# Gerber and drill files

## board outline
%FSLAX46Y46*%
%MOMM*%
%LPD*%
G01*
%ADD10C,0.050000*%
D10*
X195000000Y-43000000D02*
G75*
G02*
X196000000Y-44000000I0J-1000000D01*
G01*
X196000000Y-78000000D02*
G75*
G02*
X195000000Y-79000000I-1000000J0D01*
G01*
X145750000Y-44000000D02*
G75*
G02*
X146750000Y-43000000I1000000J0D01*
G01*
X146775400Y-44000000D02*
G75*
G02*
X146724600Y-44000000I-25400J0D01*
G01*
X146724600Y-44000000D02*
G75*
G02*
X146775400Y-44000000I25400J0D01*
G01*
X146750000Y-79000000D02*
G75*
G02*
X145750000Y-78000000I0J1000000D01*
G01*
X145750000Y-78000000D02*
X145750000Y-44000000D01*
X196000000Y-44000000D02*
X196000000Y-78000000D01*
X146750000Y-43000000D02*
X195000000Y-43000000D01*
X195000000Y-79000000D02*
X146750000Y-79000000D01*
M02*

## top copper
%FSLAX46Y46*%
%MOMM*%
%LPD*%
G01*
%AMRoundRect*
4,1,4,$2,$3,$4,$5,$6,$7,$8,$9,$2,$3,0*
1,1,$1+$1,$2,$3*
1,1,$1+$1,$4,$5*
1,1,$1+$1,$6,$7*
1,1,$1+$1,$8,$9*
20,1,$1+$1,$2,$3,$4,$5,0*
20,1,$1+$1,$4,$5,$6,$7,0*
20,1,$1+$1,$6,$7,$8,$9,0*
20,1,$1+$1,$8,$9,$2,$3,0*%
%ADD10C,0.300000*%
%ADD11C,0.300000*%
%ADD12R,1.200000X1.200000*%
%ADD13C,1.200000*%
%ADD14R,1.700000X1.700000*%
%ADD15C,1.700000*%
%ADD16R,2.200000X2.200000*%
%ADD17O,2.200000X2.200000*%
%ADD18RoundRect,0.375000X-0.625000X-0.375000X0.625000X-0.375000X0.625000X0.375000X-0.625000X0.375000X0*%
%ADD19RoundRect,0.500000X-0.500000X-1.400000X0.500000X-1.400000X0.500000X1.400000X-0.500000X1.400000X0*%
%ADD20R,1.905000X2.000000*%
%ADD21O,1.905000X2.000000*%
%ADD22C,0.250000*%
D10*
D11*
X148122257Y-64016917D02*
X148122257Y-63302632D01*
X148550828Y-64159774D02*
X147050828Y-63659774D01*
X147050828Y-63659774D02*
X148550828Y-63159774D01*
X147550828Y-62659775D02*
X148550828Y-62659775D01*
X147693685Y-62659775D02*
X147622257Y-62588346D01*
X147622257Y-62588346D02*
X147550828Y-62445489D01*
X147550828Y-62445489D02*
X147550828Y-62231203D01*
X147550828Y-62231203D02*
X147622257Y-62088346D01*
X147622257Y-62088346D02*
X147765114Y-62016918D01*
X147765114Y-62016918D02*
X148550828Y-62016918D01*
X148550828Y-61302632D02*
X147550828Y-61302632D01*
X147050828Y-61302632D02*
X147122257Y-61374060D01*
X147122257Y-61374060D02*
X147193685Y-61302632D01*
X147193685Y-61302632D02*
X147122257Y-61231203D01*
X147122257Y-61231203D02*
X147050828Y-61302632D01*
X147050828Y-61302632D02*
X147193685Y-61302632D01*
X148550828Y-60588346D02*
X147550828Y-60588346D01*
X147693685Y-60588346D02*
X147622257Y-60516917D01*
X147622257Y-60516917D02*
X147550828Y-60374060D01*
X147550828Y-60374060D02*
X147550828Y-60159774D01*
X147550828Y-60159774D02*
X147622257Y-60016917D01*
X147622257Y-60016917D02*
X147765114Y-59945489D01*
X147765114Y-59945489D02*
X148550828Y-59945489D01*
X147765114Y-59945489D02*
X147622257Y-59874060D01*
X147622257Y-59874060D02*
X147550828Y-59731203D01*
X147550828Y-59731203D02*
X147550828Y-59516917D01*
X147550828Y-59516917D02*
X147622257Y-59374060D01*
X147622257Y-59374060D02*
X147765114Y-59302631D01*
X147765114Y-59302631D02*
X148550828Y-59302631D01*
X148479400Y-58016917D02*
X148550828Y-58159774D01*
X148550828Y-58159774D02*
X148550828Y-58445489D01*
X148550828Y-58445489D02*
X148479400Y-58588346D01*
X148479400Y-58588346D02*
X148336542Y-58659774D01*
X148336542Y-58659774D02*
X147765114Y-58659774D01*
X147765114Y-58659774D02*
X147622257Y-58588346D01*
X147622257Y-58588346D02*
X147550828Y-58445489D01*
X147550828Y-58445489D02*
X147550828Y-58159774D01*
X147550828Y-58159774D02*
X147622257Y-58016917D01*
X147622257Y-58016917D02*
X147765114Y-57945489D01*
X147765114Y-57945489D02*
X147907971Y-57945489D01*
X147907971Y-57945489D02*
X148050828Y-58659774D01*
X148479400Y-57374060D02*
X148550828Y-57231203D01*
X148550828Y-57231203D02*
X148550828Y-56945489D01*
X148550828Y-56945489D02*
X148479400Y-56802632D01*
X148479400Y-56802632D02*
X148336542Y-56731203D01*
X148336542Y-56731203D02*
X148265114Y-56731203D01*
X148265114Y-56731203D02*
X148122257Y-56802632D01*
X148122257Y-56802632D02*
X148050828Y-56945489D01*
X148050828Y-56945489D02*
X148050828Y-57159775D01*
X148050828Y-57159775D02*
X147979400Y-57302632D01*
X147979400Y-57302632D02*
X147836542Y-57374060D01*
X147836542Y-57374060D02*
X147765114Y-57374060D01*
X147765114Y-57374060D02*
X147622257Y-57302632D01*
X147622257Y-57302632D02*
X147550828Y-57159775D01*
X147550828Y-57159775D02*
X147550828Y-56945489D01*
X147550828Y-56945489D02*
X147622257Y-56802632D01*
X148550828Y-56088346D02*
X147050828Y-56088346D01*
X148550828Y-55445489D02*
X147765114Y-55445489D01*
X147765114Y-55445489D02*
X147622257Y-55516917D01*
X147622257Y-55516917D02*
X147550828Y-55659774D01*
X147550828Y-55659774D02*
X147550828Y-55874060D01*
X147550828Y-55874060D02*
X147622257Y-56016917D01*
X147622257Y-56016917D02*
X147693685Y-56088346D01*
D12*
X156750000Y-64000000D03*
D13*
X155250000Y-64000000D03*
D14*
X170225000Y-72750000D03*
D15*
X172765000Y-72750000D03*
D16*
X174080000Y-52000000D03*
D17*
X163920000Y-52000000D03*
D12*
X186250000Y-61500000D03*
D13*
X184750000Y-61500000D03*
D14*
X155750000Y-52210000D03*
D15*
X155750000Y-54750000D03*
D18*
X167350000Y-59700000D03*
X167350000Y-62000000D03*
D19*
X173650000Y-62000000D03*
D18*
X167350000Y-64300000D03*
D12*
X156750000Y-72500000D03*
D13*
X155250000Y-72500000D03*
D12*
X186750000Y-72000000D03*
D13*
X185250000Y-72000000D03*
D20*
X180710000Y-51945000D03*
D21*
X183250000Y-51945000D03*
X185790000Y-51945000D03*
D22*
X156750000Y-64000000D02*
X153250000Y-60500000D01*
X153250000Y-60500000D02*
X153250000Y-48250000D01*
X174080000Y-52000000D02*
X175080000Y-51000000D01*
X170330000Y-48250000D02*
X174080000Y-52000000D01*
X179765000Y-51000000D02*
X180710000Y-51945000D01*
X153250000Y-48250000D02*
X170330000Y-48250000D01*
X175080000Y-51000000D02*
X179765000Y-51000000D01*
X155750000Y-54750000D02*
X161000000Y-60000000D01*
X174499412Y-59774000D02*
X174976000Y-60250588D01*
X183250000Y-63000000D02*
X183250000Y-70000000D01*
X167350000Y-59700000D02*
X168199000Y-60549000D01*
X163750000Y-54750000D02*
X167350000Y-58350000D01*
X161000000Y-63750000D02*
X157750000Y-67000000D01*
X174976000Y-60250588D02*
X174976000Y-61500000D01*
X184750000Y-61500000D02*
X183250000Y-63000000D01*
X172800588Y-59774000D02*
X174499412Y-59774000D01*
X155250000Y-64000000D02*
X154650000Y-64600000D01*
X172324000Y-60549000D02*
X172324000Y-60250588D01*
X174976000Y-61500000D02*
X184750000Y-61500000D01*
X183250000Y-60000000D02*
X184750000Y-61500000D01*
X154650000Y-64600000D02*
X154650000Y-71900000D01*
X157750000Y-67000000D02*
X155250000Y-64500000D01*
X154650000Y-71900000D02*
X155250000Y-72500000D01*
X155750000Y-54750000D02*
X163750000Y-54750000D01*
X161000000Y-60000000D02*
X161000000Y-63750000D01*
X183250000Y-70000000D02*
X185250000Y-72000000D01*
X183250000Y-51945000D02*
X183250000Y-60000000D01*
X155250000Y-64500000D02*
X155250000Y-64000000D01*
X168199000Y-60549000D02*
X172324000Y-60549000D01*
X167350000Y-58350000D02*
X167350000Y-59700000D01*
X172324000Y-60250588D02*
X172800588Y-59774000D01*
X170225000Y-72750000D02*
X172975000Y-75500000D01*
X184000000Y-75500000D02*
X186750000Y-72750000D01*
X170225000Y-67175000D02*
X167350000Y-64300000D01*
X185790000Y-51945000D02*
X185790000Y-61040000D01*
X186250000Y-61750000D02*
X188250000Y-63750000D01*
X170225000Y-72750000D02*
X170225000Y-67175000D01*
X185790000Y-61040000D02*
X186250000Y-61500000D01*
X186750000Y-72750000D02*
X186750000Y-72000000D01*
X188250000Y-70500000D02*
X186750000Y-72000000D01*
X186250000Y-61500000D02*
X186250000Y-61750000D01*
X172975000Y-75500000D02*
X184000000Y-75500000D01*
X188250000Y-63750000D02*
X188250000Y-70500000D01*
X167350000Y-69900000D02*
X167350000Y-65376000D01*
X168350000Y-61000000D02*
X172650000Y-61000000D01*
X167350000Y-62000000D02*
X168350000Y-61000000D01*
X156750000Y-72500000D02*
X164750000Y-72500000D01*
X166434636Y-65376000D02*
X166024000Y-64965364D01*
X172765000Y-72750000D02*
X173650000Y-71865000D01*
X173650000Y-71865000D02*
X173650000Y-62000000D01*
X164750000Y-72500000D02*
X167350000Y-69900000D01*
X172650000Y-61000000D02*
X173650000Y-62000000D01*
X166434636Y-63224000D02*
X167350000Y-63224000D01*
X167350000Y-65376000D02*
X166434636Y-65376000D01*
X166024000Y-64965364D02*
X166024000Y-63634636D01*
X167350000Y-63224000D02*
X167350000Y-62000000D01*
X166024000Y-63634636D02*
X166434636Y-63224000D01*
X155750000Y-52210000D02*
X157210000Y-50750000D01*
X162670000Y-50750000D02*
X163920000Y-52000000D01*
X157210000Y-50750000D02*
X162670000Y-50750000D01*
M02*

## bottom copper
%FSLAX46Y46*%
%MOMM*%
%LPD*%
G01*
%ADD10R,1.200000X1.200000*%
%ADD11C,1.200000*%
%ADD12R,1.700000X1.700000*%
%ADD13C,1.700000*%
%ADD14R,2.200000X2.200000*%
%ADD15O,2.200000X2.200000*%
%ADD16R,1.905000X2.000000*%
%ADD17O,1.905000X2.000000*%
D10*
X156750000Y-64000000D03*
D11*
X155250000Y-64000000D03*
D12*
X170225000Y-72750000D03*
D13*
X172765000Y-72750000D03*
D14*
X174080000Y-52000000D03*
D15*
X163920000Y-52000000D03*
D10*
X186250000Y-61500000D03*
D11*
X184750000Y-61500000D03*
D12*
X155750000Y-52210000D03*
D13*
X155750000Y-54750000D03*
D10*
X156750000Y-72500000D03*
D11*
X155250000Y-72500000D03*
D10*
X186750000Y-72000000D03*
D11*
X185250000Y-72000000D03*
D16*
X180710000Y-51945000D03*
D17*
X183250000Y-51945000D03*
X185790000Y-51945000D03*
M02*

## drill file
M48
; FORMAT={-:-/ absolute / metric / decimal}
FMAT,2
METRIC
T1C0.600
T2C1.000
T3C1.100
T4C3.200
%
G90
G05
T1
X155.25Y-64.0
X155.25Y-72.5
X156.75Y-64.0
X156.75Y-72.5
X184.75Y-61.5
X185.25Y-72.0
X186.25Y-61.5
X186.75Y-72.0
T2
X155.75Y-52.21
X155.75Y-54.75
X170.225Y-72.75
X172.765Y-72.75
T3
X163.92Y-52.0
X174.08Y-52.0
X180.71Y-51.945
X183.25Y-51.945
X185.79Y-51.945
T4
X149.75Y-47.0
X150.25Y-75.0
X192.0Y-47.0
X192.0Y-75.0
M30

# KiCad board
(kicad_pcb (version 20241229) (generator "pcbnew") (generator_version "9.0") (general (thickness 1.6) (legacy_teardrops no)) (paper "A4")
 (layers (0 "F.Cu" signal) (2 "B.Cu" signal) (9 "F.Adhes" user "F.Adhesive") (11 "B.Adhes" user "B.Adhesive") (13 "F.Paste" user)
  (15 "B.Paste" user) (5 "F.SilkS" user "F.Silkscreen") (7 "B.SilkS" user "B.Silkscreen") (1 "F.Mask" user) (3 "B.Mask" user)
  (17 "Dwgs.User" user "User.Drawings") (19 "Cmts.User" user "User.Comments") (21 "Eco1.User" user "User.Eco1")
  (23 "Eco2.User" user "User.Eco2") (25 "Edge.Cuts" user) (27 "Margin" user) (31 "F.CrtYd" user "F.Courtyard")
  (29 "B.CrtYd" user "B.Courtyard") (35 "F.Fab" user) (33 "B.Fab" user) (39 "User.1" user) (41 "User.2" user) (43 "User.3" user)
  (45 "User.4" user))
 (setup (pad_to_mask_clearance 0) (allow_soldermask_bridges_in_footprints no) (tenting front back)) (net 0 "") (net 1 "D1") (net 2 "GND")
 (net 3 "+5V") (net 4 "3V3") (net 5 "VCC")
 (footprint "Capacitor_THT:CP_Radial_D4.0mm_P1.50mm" (layer "F.Cu") (at 156.75 64 180)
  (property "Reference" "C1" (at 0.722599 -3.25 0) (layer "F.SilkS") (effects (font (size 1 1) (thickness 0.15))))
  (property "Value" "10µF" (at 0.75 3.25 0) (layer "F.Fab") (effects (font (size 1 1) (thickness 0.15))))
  (pad "1" thru_hole rect (at 0 0 180) (size 1.2 1.2) (drill 0.6) (layers "*.Cu" "*.Mask") (remove_unused_layers no) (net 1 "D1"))
  (pad "2" thru_hole circle (at 1.5 0 180) (size 1.2 1.2) (drill 0.6) (layers "*.Cu" "*.Mask") (remove_unused_layers no) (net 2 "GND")))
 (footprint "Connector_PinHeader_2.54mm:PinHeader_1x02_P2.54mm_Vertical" (layer "F.Cu") (at 170.225 72.75 90)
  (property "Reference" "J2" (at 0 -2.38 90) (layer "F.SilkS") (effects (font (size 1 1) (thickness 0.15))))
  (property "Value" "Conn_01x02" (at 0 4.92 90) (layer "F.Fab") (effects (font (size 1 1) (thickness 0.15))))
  (pad "1" thru_hole rect (at 0 0 90) (size 1.7 1.7) (drill 1) (layers "*.Cu" "*.Mask") (remove_unused_layers no) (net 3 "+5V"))
  (pad "2" thru_hole circle (at 0 2.54 90) (size 1.7 1.7) (drill 1) (layers "*.Cu" "*.Mask") (remove_unused_layers no) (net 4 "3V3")))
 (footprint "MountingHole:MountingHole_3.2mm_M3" (layer "F.Cu") (at 150.25 75)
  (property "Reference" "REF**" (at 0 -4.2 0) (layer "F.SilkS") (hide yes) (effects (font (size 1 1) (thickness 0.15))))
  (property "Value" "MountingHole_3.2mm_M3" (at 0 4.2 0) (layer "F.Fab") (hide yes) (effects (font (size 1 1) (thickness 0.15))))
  (pad "" np_thru_hole circle (at 0 0) (size 3.2 3.2) (drill 3.2) (layers "*.Cu" "*.Mask")))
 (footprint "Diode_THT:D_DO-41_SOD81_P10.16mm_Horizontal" (layer "F.Cu") (at 174.08 52 180)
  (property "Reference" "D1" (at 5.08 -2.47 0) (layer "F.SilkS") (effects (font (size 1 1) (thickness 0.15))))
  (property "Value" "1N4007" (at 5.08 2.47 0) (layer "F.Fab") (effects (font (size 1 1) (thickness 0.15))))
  (pad "1" thru_hole rect (at 0 0 180) (size 2.2 2.2) (drill 1.1) (layers "*.Cu" "*.Mask") (remove_unused_layers no) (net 1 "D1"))
  (pad "2" thru_hole oval (at 10.16 0 180) (size 2.2 2.2) (drill 1.1) (layers "*.Cu" "*.Mask") (remove_unused_layers no) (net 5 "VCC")))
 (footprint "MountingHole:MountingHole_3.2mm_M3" (layer "F.Cu") (at 149.75 47)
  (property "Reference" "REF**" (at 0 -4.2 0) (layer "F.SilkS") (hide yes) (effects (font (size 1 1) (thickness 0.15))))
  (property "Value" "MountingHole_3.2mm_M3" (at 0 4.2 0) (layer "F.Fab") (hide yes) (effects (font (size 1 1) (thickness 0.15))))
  (pad "" np_thru_hole circle (at 0 0) (size 3.2 3.2) (drill 3.2) (layers "*.Cu" "*.Mask")))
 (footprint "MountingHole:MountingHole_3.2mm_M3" (layer "F.Cu") (at 192 47)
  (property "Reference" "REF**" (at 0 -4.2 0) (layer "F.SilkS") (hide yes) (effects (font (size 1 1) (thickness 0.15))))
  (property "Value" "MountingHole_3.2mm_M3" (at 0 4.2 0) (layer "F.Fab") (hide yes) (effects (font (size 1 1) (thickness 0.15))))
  (pad "" np_thru_hole circle (at 0 0) (size 3.2 3.2) (drill 3.2) (layers "*.Cu" "*.Mask")))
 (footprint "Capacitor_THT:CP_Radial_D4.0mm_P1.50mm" (layer "F.Cu") (at 186.25 61.5 180)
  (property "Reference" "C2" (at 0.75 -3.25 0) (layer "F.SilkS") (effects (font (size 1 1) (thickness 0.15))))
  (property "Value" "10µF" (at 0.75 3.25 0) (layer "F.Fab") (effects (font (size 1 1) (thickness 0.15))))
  (pad "1" thru_hole rect (at 0 0 180) (size 1.2 1.2) (drill 0.6) (layers "*.Cu" "*.Mask") (remove_unused_layers no) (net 3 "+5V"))
  (pad "2" thru_hole circle (at 1.5 0 180) (size 1.2 1.2) (drill 0.6) (layers "*.Cu" "*.Mask") (remove_unused_layers no) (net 2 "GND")))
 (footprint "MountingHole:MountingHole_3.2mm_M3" (layer "F.Cu") (at 192 75)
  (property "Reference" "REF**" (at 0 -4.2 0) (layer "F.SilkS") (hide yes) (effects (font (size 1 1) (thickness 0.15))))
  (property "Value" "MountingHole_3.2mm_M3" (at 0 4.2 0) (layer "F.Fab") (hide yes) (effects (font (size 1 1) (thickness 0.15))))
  (pad "" np_thru_hole circle (at 0 0) (size 3.2 3.2) (drill 3.2) (layers "*.Cu" "*.Mask")))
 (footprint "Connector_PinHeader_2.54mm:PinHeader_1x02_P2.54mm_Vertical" (layer "F.Cu") (at 155.75 52.21)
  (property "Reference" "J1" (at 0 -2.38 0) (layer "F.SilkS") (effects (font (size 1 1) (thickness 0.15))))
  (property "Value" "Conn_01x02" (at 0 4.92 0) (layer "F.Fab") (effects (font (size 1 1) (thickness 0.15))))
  (pad "1" thru_hole rect (at 0 0) (size 1.7 1.7) (drill 1) (layers "*.Cu" "*.Mask") (remove_unused_layers no) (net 5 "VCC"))
  (pad "2" thru_hole circle (at 0 2.54) (size 1.7 1.7) (drill 1) (layers "*.Cu" "*.Mask") (remove_unused_layers no) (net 2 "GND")))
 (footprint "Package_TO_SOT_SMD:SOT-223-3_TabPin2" (layer "F.Cu") (at 170.5 62)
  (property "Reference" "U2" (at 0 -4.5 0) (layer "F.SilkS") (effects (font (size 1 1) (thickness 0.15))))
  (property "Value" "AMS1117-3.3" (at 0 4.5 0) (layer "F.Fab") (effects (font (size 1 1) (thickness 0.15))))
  (pad "1" smd roundrect (at -3.15 -2.3) (size 2 1.5) (layers "F.Cu" "F.Mask" "F.Paste") (roundrect_rratio 0.25) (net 2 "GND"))
  (pad "2" smd roundrect (at -3.15 0) (size 2 1.5) (layers "F.Cu" "F.Mask" "F.Paste") (roundrect_rratio 0.25) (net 4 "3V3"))
  (pad "2" smd roundrect (at 3.15 0) (size 2 3.8) (layers "F.Cu" "F.Mask" "F.Paste") (roundrect_rratio 0.25) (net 4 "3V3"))
  (pad "3" smd roundrect (at -3.15 2.3) (size 2 1.5) (layers "F.Cu" "F.Mask" "F.Paste") (roundrect_rratio 0.25) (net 3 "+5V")))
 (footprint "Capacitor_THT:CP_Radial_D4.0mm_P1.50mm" (layer "F.Cu") (at 156.75 72.5 180)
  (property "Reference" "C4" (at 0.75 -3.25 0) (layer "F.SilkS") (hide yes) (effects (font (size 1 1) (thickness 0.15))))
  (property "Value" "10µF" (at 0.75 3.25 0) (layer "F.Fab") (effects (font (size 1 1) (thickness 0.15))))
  (pad "1" thru_hole rect (at 0 0 180) (size 1.2 1.2) (drill 0.6) (layers "*.Cu" "*.Mask") (remove_unused_layers no) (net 4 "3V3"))
  (pad "2" thru_hole circle (at 1.5 0 180) (size 1.2 1.2) (drill 0.6) (layers "*.Cu" "*.Mask") (remove_unused_layers no) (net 2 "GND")))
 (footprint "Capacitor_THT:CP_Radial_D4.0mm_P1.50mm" (layer "F.Cu") (at 186.75 72 180)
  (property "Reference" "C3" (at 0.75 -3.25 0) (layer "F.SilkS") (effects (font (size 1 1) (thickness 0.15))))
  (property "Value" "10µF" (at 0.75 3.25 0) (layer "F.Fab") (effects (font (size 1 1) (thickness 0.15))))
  (pad "1" thru_hole rect (at 0 0 180) (size 1.2 1.2) (drill 0.6) (layers "*.Cu" "*.Mask") (remove_unused_layers no) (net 3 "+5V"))
  (pad "2" thru_hole circle (at 1.5 0 180) (size 1.2 1.2) (drill 0.6) (layers "*.Cu" "*.Mask") (remove_unused_layers no) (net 2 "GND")))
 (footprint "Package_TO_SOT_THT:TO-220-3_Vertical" (layer "F.Cu") (at 180.71 51.945)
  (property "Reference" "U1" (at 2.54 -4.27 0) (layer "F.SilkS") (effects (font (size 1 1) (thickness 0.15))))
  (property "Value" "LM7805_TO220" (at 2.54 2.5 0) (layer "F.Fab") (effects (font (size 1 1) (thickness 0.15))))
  (pad "1" thru_hole rect (at 0 0) (size 1.905 2) (drill 1.1) (layers "*.Cu" "*.Mask") (remove_unused_layers no) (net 1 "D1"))
  (pad "2" thru_hole oval (at 2.54 0) (size 1.905 2) (drill 1.1) (layers "*.Cu" "*.Mask") (remove_unused_layers no) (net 2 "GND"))
  (pad "3" thru_hole oval (at 5.08 0) (size 1.905 2) (drill 1.1) (layers "*.Cu" "*.Mask") (remove_unused_layers no) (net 3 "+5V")))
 (gr_arc (start 195 43) (mid 195.707107 43.292893) (end 196 44) (stroke (width 0.05) (type default)) (layer "Edge.Cuts"))
 (gr_arc (start 196 78) (mid 195.707107 78.707107) (end 195 79) (stroke (width 0.05) (type default)) (layer "Edge.Cuts"))
 (gr_arc (start 145.75 44) (mid 146.042893 43.292893) (end 146.75 43) (stroke (width 0.05) (type default)) (layer "Edge.Cuts"))
 (gr_arc (start 146.7246 44) (mid 146.7754 44) (end 146.7246 44) (stroke (width 0.05) (type default)) (layer "Edge.Cuts"))
 (gr_arc (start 146.75 79) (mid 146.042893 78.707107) (end 145.75 78) (stroke (width 0.05) (type default)) (layer "Edge.Cuts"))
 (gr_line (start 145.75 78) (end 145.75 44) (stroke (width 0.05) (type default)) (layer "Edge.Cuts"))
 (gr_line (start 196 44) (end 196 78) (stroke (width 0.05) (type default)) (layer "Edge.Cuts"))
 (gr_line (start 146.75 43) (end 195 43) (stroke (width 0.05) (type default)) (layer "Edge.Cuts"))
 (gr_line (start 195 79) (end 146.75 79) (stroke (width 0.05) (type default)) (layer "Edge.Cuts"))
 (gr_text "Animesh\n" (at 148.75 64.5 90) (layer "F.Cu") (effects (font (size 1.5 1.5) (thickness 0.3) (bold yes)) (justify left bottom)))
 (segment (start 156.75 64) (end 153.25 60.5) (width 0.25) (layer "F.Cu") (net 1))
 (segment (start 153.25 60.5) (end 153.25 48.25) (width 0.25) (layer "F.Cu") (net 1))
 (segment (start 174.08 52) (end 175.08 51) (width 0.25) (layer "F.Cu") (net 1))
 (segment (start 170.33 48.25) (end 174.08 52) (width 0.25) (layer "F.Cu") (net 1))
 (segment (start 179.765 51) (end 180.71 51.945) (width 0.25) (layer "F.Cu") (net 1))
 (segment (start 153.25 48.25) (end 170.33 48.25) (width 0.25) (layer "F.Cu") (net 1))
 (segment (start 175.08 51) (end 179.765 51) (width 0.25) (layer "F.Cu") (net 1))
 (segment (start 155.75 54.75) (end 161 60) (width 0.25) (layer "F.Cu") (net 2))
 (segment (start 174.499412 59.774) (end 174.976 60.250588) (width 0.25) (layer "F.Cu") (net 2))
 (segment (start 183.25 63) (end 183.25 70) (width 0.25) (layer "F.Cu") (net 2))
 (segment (start 167.35 59.7) (end 168.199 60.549) (width 0.25) (layer "F.Cu") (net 2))
 (segment (start 163.75 54.75) (end 167.35 58.35) (width 0.25) (layer "F.Cu") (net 2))
 (segment (start 161 63.75) (end 157.75 67) (width 0.25) (layer "F.Cu") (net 2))
 (segment (start 174.976 60.250588) (end 174.976 61.5) (width 0.25) (layer "F.Cu") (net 2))
 (segment (start 184.75 61.5) (end 183.25 63) (width 0.25) (layer "F.Cu") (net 2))
 (segment (start 172.800588 59.774) (end 174.499412 59.774) (width 0.25) (layer "F.Cu") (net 2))
 (segment (start 155.25 64) (end 154.65 64.6) (width 0.25) (layer "F.Cu") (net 2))
 (segment (start 172.324 60.549) (end 172.324 60.250588) (width 0.25) (layer "F.Cu") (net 2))
 (segment (start 174.976 61.5) (end 184.75 61.5) (width 0.25) (layer "F.Cu") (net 2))
 (segment (start 183.25 60) (end 184.75 61.5) (width 0.25) (layer "F.Cu") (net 2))
 (segment (start 154.65 64.6) (end 154.65 71.9) (width 0.25) (layer "F.Cu") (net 2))
 (segment (start 157.75 67) (end 155.25 64.5) (width 0.25) (layer "F.Cu") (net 2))
 (segment (start 154.65 71.9) (end 155.25 72.5) (width 0.25) (layer "F.Cu") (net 2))
 (segment (start 155.75 54.75) (end 163.75 54.75) (width 0.25) (layer "F.Cu") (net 2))
 (segment (start 161 60) (end 161 63.75) (width 0.25) (layer "F.Cu") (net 2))
 (segment (start 183.25 70) (end 185.25 72) (width 0.25) (layer "F.Cu") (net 2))
 (segment (start 183.25 51.945) (end 183.25 60) (width 0.25) (layer "F.Cu") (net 2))
 (segment (start 155.25 64.5) (end 155.25 64) (width 0.25) (layer "F.Cu") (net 2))
 (segment (start 168.199 60.549) (end 172.324 60.549) (width 0.25) (layer "F.Cu") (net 2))
 (segment (start 167.35 58.35) (end 167.35 59.7) (width 0.25) (layer "F.Cu") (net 2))
 (segment (start 172.324 60.250588) (end 172.800588 59.774) (width 0.25) (layer "F.Cu") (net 2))
 (segment (start 170.225 72.75) (end 172.975 75.5) (width 0.25) (layer "F.Cu") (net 3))
 (segment (start 184 75.5) (end 186.75 72.75) (width 0.25) (layer "F.Cu") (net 3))
 (segment (start 170.225 67.175) (end 167.35 64.3) (width 0.25) (layer "F.Cu") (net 3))
 (segment (start 185.79 51.945) (end 185.79 61.04) (width 0.25) (layer "F.Cu") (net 3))
 (segment (start 186.25 61.75) (end 188.25 63.75) (width 0.25) (layer "F.Cu") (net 3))
 (segment (start 170.225 72.75) (end 170.225 67.175) (width 0.25) (layer "F.Cu") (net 3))
 (segment (start 185.79 61.04) (end 186.25 61.5) (width 0.25) (layer "F.Cu") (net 3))
 (segment (start 186.75 72.75) (end 186.75 72) (width 0.25) (layer "F.Cu") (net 3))
 (segment (start 188.25 70.5) (end 186.75 72) (width 0.25) (layer "F.Cu") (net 3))
 (segment (start 186.25 61.5) (end 186.25 61.75) (width 0.25) (layer "F.Cu") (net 3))
 (segment (start 172.975 75.5) (end 184 75.5) (width 0.25) (layer "F.Cu") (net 3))
 (segment (start 188.25 63.75) (end 188.25 70.5) (width 0.25) (layer "F.Cu") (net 3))
 (segment (start 167.35 69.9) (end 167.35 65.376) (width 0.25) (layer "F.Cu") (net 4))
 (segment (start 168.35 61) (end 172.65 61) (width 0.25) (layer "F.Cu") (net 4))
 (segment (start 167.35 62) (end 168.35 61) (width 0.25) (layer "F.Cu") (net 4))
 (segment (start 156.75 72.5) (end 164.75 72.5) (width 0.25) (layer "F.Cu") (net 4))
 (segment (start 166.434636 65.376) (end 166.024 64.965364) (width 0.25) (layer "F.Cu") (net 4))
 (segment (start 172.765 72.75) (end 173.65 71.865) (width 0.25) (layer "F.Cu") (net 4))
 (segment (start 173.65 71.865) (end 173.65 62) (width 0.25) (layer "F.Cu") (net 4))
 (segment (start 164.75 72.5) (end 167.35 69.9) (width 0.25) (layer "F.Cu") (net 4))
 (segment (start 172.65 61) (end 173.65 62) (width 0.25) (layer "F.Cu") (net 4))
 (segment (start 166.434636 63.224) (end 167.35 63.224) (width 0.25) (layer "F.Cu") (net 4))
 (segment (start 167.35 65.376) (end 166.434636 65.376) (width 0.25) (layer "F.Cu") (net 4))
 (segment (start 166.024 64.965364) (end 166.024 63.634636) (width 0.25) (layer "F.Cu") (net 4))
 (segment (start 167.35 63.224) (end 167.35 62) (width 0.25) (layer "F.Cu") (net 4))
 (segment (start 166.024 63.634636) (end 166.434636 63.224) (width 0.25) (layer "F.Cu") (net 4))
 (segment (start 155.75 52.21) (end 157.21 50.75) (width 0.25) (layer "F.Cu") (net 5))
 (segment (start 162.67 50.75) (end 163.92 52) (width 0.25) (layer "F.Cu") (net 5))
 (segment (start 157.21 50.75) (end 162.67 50.75) (width 0.25) (layer "F.Cu") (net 5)))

